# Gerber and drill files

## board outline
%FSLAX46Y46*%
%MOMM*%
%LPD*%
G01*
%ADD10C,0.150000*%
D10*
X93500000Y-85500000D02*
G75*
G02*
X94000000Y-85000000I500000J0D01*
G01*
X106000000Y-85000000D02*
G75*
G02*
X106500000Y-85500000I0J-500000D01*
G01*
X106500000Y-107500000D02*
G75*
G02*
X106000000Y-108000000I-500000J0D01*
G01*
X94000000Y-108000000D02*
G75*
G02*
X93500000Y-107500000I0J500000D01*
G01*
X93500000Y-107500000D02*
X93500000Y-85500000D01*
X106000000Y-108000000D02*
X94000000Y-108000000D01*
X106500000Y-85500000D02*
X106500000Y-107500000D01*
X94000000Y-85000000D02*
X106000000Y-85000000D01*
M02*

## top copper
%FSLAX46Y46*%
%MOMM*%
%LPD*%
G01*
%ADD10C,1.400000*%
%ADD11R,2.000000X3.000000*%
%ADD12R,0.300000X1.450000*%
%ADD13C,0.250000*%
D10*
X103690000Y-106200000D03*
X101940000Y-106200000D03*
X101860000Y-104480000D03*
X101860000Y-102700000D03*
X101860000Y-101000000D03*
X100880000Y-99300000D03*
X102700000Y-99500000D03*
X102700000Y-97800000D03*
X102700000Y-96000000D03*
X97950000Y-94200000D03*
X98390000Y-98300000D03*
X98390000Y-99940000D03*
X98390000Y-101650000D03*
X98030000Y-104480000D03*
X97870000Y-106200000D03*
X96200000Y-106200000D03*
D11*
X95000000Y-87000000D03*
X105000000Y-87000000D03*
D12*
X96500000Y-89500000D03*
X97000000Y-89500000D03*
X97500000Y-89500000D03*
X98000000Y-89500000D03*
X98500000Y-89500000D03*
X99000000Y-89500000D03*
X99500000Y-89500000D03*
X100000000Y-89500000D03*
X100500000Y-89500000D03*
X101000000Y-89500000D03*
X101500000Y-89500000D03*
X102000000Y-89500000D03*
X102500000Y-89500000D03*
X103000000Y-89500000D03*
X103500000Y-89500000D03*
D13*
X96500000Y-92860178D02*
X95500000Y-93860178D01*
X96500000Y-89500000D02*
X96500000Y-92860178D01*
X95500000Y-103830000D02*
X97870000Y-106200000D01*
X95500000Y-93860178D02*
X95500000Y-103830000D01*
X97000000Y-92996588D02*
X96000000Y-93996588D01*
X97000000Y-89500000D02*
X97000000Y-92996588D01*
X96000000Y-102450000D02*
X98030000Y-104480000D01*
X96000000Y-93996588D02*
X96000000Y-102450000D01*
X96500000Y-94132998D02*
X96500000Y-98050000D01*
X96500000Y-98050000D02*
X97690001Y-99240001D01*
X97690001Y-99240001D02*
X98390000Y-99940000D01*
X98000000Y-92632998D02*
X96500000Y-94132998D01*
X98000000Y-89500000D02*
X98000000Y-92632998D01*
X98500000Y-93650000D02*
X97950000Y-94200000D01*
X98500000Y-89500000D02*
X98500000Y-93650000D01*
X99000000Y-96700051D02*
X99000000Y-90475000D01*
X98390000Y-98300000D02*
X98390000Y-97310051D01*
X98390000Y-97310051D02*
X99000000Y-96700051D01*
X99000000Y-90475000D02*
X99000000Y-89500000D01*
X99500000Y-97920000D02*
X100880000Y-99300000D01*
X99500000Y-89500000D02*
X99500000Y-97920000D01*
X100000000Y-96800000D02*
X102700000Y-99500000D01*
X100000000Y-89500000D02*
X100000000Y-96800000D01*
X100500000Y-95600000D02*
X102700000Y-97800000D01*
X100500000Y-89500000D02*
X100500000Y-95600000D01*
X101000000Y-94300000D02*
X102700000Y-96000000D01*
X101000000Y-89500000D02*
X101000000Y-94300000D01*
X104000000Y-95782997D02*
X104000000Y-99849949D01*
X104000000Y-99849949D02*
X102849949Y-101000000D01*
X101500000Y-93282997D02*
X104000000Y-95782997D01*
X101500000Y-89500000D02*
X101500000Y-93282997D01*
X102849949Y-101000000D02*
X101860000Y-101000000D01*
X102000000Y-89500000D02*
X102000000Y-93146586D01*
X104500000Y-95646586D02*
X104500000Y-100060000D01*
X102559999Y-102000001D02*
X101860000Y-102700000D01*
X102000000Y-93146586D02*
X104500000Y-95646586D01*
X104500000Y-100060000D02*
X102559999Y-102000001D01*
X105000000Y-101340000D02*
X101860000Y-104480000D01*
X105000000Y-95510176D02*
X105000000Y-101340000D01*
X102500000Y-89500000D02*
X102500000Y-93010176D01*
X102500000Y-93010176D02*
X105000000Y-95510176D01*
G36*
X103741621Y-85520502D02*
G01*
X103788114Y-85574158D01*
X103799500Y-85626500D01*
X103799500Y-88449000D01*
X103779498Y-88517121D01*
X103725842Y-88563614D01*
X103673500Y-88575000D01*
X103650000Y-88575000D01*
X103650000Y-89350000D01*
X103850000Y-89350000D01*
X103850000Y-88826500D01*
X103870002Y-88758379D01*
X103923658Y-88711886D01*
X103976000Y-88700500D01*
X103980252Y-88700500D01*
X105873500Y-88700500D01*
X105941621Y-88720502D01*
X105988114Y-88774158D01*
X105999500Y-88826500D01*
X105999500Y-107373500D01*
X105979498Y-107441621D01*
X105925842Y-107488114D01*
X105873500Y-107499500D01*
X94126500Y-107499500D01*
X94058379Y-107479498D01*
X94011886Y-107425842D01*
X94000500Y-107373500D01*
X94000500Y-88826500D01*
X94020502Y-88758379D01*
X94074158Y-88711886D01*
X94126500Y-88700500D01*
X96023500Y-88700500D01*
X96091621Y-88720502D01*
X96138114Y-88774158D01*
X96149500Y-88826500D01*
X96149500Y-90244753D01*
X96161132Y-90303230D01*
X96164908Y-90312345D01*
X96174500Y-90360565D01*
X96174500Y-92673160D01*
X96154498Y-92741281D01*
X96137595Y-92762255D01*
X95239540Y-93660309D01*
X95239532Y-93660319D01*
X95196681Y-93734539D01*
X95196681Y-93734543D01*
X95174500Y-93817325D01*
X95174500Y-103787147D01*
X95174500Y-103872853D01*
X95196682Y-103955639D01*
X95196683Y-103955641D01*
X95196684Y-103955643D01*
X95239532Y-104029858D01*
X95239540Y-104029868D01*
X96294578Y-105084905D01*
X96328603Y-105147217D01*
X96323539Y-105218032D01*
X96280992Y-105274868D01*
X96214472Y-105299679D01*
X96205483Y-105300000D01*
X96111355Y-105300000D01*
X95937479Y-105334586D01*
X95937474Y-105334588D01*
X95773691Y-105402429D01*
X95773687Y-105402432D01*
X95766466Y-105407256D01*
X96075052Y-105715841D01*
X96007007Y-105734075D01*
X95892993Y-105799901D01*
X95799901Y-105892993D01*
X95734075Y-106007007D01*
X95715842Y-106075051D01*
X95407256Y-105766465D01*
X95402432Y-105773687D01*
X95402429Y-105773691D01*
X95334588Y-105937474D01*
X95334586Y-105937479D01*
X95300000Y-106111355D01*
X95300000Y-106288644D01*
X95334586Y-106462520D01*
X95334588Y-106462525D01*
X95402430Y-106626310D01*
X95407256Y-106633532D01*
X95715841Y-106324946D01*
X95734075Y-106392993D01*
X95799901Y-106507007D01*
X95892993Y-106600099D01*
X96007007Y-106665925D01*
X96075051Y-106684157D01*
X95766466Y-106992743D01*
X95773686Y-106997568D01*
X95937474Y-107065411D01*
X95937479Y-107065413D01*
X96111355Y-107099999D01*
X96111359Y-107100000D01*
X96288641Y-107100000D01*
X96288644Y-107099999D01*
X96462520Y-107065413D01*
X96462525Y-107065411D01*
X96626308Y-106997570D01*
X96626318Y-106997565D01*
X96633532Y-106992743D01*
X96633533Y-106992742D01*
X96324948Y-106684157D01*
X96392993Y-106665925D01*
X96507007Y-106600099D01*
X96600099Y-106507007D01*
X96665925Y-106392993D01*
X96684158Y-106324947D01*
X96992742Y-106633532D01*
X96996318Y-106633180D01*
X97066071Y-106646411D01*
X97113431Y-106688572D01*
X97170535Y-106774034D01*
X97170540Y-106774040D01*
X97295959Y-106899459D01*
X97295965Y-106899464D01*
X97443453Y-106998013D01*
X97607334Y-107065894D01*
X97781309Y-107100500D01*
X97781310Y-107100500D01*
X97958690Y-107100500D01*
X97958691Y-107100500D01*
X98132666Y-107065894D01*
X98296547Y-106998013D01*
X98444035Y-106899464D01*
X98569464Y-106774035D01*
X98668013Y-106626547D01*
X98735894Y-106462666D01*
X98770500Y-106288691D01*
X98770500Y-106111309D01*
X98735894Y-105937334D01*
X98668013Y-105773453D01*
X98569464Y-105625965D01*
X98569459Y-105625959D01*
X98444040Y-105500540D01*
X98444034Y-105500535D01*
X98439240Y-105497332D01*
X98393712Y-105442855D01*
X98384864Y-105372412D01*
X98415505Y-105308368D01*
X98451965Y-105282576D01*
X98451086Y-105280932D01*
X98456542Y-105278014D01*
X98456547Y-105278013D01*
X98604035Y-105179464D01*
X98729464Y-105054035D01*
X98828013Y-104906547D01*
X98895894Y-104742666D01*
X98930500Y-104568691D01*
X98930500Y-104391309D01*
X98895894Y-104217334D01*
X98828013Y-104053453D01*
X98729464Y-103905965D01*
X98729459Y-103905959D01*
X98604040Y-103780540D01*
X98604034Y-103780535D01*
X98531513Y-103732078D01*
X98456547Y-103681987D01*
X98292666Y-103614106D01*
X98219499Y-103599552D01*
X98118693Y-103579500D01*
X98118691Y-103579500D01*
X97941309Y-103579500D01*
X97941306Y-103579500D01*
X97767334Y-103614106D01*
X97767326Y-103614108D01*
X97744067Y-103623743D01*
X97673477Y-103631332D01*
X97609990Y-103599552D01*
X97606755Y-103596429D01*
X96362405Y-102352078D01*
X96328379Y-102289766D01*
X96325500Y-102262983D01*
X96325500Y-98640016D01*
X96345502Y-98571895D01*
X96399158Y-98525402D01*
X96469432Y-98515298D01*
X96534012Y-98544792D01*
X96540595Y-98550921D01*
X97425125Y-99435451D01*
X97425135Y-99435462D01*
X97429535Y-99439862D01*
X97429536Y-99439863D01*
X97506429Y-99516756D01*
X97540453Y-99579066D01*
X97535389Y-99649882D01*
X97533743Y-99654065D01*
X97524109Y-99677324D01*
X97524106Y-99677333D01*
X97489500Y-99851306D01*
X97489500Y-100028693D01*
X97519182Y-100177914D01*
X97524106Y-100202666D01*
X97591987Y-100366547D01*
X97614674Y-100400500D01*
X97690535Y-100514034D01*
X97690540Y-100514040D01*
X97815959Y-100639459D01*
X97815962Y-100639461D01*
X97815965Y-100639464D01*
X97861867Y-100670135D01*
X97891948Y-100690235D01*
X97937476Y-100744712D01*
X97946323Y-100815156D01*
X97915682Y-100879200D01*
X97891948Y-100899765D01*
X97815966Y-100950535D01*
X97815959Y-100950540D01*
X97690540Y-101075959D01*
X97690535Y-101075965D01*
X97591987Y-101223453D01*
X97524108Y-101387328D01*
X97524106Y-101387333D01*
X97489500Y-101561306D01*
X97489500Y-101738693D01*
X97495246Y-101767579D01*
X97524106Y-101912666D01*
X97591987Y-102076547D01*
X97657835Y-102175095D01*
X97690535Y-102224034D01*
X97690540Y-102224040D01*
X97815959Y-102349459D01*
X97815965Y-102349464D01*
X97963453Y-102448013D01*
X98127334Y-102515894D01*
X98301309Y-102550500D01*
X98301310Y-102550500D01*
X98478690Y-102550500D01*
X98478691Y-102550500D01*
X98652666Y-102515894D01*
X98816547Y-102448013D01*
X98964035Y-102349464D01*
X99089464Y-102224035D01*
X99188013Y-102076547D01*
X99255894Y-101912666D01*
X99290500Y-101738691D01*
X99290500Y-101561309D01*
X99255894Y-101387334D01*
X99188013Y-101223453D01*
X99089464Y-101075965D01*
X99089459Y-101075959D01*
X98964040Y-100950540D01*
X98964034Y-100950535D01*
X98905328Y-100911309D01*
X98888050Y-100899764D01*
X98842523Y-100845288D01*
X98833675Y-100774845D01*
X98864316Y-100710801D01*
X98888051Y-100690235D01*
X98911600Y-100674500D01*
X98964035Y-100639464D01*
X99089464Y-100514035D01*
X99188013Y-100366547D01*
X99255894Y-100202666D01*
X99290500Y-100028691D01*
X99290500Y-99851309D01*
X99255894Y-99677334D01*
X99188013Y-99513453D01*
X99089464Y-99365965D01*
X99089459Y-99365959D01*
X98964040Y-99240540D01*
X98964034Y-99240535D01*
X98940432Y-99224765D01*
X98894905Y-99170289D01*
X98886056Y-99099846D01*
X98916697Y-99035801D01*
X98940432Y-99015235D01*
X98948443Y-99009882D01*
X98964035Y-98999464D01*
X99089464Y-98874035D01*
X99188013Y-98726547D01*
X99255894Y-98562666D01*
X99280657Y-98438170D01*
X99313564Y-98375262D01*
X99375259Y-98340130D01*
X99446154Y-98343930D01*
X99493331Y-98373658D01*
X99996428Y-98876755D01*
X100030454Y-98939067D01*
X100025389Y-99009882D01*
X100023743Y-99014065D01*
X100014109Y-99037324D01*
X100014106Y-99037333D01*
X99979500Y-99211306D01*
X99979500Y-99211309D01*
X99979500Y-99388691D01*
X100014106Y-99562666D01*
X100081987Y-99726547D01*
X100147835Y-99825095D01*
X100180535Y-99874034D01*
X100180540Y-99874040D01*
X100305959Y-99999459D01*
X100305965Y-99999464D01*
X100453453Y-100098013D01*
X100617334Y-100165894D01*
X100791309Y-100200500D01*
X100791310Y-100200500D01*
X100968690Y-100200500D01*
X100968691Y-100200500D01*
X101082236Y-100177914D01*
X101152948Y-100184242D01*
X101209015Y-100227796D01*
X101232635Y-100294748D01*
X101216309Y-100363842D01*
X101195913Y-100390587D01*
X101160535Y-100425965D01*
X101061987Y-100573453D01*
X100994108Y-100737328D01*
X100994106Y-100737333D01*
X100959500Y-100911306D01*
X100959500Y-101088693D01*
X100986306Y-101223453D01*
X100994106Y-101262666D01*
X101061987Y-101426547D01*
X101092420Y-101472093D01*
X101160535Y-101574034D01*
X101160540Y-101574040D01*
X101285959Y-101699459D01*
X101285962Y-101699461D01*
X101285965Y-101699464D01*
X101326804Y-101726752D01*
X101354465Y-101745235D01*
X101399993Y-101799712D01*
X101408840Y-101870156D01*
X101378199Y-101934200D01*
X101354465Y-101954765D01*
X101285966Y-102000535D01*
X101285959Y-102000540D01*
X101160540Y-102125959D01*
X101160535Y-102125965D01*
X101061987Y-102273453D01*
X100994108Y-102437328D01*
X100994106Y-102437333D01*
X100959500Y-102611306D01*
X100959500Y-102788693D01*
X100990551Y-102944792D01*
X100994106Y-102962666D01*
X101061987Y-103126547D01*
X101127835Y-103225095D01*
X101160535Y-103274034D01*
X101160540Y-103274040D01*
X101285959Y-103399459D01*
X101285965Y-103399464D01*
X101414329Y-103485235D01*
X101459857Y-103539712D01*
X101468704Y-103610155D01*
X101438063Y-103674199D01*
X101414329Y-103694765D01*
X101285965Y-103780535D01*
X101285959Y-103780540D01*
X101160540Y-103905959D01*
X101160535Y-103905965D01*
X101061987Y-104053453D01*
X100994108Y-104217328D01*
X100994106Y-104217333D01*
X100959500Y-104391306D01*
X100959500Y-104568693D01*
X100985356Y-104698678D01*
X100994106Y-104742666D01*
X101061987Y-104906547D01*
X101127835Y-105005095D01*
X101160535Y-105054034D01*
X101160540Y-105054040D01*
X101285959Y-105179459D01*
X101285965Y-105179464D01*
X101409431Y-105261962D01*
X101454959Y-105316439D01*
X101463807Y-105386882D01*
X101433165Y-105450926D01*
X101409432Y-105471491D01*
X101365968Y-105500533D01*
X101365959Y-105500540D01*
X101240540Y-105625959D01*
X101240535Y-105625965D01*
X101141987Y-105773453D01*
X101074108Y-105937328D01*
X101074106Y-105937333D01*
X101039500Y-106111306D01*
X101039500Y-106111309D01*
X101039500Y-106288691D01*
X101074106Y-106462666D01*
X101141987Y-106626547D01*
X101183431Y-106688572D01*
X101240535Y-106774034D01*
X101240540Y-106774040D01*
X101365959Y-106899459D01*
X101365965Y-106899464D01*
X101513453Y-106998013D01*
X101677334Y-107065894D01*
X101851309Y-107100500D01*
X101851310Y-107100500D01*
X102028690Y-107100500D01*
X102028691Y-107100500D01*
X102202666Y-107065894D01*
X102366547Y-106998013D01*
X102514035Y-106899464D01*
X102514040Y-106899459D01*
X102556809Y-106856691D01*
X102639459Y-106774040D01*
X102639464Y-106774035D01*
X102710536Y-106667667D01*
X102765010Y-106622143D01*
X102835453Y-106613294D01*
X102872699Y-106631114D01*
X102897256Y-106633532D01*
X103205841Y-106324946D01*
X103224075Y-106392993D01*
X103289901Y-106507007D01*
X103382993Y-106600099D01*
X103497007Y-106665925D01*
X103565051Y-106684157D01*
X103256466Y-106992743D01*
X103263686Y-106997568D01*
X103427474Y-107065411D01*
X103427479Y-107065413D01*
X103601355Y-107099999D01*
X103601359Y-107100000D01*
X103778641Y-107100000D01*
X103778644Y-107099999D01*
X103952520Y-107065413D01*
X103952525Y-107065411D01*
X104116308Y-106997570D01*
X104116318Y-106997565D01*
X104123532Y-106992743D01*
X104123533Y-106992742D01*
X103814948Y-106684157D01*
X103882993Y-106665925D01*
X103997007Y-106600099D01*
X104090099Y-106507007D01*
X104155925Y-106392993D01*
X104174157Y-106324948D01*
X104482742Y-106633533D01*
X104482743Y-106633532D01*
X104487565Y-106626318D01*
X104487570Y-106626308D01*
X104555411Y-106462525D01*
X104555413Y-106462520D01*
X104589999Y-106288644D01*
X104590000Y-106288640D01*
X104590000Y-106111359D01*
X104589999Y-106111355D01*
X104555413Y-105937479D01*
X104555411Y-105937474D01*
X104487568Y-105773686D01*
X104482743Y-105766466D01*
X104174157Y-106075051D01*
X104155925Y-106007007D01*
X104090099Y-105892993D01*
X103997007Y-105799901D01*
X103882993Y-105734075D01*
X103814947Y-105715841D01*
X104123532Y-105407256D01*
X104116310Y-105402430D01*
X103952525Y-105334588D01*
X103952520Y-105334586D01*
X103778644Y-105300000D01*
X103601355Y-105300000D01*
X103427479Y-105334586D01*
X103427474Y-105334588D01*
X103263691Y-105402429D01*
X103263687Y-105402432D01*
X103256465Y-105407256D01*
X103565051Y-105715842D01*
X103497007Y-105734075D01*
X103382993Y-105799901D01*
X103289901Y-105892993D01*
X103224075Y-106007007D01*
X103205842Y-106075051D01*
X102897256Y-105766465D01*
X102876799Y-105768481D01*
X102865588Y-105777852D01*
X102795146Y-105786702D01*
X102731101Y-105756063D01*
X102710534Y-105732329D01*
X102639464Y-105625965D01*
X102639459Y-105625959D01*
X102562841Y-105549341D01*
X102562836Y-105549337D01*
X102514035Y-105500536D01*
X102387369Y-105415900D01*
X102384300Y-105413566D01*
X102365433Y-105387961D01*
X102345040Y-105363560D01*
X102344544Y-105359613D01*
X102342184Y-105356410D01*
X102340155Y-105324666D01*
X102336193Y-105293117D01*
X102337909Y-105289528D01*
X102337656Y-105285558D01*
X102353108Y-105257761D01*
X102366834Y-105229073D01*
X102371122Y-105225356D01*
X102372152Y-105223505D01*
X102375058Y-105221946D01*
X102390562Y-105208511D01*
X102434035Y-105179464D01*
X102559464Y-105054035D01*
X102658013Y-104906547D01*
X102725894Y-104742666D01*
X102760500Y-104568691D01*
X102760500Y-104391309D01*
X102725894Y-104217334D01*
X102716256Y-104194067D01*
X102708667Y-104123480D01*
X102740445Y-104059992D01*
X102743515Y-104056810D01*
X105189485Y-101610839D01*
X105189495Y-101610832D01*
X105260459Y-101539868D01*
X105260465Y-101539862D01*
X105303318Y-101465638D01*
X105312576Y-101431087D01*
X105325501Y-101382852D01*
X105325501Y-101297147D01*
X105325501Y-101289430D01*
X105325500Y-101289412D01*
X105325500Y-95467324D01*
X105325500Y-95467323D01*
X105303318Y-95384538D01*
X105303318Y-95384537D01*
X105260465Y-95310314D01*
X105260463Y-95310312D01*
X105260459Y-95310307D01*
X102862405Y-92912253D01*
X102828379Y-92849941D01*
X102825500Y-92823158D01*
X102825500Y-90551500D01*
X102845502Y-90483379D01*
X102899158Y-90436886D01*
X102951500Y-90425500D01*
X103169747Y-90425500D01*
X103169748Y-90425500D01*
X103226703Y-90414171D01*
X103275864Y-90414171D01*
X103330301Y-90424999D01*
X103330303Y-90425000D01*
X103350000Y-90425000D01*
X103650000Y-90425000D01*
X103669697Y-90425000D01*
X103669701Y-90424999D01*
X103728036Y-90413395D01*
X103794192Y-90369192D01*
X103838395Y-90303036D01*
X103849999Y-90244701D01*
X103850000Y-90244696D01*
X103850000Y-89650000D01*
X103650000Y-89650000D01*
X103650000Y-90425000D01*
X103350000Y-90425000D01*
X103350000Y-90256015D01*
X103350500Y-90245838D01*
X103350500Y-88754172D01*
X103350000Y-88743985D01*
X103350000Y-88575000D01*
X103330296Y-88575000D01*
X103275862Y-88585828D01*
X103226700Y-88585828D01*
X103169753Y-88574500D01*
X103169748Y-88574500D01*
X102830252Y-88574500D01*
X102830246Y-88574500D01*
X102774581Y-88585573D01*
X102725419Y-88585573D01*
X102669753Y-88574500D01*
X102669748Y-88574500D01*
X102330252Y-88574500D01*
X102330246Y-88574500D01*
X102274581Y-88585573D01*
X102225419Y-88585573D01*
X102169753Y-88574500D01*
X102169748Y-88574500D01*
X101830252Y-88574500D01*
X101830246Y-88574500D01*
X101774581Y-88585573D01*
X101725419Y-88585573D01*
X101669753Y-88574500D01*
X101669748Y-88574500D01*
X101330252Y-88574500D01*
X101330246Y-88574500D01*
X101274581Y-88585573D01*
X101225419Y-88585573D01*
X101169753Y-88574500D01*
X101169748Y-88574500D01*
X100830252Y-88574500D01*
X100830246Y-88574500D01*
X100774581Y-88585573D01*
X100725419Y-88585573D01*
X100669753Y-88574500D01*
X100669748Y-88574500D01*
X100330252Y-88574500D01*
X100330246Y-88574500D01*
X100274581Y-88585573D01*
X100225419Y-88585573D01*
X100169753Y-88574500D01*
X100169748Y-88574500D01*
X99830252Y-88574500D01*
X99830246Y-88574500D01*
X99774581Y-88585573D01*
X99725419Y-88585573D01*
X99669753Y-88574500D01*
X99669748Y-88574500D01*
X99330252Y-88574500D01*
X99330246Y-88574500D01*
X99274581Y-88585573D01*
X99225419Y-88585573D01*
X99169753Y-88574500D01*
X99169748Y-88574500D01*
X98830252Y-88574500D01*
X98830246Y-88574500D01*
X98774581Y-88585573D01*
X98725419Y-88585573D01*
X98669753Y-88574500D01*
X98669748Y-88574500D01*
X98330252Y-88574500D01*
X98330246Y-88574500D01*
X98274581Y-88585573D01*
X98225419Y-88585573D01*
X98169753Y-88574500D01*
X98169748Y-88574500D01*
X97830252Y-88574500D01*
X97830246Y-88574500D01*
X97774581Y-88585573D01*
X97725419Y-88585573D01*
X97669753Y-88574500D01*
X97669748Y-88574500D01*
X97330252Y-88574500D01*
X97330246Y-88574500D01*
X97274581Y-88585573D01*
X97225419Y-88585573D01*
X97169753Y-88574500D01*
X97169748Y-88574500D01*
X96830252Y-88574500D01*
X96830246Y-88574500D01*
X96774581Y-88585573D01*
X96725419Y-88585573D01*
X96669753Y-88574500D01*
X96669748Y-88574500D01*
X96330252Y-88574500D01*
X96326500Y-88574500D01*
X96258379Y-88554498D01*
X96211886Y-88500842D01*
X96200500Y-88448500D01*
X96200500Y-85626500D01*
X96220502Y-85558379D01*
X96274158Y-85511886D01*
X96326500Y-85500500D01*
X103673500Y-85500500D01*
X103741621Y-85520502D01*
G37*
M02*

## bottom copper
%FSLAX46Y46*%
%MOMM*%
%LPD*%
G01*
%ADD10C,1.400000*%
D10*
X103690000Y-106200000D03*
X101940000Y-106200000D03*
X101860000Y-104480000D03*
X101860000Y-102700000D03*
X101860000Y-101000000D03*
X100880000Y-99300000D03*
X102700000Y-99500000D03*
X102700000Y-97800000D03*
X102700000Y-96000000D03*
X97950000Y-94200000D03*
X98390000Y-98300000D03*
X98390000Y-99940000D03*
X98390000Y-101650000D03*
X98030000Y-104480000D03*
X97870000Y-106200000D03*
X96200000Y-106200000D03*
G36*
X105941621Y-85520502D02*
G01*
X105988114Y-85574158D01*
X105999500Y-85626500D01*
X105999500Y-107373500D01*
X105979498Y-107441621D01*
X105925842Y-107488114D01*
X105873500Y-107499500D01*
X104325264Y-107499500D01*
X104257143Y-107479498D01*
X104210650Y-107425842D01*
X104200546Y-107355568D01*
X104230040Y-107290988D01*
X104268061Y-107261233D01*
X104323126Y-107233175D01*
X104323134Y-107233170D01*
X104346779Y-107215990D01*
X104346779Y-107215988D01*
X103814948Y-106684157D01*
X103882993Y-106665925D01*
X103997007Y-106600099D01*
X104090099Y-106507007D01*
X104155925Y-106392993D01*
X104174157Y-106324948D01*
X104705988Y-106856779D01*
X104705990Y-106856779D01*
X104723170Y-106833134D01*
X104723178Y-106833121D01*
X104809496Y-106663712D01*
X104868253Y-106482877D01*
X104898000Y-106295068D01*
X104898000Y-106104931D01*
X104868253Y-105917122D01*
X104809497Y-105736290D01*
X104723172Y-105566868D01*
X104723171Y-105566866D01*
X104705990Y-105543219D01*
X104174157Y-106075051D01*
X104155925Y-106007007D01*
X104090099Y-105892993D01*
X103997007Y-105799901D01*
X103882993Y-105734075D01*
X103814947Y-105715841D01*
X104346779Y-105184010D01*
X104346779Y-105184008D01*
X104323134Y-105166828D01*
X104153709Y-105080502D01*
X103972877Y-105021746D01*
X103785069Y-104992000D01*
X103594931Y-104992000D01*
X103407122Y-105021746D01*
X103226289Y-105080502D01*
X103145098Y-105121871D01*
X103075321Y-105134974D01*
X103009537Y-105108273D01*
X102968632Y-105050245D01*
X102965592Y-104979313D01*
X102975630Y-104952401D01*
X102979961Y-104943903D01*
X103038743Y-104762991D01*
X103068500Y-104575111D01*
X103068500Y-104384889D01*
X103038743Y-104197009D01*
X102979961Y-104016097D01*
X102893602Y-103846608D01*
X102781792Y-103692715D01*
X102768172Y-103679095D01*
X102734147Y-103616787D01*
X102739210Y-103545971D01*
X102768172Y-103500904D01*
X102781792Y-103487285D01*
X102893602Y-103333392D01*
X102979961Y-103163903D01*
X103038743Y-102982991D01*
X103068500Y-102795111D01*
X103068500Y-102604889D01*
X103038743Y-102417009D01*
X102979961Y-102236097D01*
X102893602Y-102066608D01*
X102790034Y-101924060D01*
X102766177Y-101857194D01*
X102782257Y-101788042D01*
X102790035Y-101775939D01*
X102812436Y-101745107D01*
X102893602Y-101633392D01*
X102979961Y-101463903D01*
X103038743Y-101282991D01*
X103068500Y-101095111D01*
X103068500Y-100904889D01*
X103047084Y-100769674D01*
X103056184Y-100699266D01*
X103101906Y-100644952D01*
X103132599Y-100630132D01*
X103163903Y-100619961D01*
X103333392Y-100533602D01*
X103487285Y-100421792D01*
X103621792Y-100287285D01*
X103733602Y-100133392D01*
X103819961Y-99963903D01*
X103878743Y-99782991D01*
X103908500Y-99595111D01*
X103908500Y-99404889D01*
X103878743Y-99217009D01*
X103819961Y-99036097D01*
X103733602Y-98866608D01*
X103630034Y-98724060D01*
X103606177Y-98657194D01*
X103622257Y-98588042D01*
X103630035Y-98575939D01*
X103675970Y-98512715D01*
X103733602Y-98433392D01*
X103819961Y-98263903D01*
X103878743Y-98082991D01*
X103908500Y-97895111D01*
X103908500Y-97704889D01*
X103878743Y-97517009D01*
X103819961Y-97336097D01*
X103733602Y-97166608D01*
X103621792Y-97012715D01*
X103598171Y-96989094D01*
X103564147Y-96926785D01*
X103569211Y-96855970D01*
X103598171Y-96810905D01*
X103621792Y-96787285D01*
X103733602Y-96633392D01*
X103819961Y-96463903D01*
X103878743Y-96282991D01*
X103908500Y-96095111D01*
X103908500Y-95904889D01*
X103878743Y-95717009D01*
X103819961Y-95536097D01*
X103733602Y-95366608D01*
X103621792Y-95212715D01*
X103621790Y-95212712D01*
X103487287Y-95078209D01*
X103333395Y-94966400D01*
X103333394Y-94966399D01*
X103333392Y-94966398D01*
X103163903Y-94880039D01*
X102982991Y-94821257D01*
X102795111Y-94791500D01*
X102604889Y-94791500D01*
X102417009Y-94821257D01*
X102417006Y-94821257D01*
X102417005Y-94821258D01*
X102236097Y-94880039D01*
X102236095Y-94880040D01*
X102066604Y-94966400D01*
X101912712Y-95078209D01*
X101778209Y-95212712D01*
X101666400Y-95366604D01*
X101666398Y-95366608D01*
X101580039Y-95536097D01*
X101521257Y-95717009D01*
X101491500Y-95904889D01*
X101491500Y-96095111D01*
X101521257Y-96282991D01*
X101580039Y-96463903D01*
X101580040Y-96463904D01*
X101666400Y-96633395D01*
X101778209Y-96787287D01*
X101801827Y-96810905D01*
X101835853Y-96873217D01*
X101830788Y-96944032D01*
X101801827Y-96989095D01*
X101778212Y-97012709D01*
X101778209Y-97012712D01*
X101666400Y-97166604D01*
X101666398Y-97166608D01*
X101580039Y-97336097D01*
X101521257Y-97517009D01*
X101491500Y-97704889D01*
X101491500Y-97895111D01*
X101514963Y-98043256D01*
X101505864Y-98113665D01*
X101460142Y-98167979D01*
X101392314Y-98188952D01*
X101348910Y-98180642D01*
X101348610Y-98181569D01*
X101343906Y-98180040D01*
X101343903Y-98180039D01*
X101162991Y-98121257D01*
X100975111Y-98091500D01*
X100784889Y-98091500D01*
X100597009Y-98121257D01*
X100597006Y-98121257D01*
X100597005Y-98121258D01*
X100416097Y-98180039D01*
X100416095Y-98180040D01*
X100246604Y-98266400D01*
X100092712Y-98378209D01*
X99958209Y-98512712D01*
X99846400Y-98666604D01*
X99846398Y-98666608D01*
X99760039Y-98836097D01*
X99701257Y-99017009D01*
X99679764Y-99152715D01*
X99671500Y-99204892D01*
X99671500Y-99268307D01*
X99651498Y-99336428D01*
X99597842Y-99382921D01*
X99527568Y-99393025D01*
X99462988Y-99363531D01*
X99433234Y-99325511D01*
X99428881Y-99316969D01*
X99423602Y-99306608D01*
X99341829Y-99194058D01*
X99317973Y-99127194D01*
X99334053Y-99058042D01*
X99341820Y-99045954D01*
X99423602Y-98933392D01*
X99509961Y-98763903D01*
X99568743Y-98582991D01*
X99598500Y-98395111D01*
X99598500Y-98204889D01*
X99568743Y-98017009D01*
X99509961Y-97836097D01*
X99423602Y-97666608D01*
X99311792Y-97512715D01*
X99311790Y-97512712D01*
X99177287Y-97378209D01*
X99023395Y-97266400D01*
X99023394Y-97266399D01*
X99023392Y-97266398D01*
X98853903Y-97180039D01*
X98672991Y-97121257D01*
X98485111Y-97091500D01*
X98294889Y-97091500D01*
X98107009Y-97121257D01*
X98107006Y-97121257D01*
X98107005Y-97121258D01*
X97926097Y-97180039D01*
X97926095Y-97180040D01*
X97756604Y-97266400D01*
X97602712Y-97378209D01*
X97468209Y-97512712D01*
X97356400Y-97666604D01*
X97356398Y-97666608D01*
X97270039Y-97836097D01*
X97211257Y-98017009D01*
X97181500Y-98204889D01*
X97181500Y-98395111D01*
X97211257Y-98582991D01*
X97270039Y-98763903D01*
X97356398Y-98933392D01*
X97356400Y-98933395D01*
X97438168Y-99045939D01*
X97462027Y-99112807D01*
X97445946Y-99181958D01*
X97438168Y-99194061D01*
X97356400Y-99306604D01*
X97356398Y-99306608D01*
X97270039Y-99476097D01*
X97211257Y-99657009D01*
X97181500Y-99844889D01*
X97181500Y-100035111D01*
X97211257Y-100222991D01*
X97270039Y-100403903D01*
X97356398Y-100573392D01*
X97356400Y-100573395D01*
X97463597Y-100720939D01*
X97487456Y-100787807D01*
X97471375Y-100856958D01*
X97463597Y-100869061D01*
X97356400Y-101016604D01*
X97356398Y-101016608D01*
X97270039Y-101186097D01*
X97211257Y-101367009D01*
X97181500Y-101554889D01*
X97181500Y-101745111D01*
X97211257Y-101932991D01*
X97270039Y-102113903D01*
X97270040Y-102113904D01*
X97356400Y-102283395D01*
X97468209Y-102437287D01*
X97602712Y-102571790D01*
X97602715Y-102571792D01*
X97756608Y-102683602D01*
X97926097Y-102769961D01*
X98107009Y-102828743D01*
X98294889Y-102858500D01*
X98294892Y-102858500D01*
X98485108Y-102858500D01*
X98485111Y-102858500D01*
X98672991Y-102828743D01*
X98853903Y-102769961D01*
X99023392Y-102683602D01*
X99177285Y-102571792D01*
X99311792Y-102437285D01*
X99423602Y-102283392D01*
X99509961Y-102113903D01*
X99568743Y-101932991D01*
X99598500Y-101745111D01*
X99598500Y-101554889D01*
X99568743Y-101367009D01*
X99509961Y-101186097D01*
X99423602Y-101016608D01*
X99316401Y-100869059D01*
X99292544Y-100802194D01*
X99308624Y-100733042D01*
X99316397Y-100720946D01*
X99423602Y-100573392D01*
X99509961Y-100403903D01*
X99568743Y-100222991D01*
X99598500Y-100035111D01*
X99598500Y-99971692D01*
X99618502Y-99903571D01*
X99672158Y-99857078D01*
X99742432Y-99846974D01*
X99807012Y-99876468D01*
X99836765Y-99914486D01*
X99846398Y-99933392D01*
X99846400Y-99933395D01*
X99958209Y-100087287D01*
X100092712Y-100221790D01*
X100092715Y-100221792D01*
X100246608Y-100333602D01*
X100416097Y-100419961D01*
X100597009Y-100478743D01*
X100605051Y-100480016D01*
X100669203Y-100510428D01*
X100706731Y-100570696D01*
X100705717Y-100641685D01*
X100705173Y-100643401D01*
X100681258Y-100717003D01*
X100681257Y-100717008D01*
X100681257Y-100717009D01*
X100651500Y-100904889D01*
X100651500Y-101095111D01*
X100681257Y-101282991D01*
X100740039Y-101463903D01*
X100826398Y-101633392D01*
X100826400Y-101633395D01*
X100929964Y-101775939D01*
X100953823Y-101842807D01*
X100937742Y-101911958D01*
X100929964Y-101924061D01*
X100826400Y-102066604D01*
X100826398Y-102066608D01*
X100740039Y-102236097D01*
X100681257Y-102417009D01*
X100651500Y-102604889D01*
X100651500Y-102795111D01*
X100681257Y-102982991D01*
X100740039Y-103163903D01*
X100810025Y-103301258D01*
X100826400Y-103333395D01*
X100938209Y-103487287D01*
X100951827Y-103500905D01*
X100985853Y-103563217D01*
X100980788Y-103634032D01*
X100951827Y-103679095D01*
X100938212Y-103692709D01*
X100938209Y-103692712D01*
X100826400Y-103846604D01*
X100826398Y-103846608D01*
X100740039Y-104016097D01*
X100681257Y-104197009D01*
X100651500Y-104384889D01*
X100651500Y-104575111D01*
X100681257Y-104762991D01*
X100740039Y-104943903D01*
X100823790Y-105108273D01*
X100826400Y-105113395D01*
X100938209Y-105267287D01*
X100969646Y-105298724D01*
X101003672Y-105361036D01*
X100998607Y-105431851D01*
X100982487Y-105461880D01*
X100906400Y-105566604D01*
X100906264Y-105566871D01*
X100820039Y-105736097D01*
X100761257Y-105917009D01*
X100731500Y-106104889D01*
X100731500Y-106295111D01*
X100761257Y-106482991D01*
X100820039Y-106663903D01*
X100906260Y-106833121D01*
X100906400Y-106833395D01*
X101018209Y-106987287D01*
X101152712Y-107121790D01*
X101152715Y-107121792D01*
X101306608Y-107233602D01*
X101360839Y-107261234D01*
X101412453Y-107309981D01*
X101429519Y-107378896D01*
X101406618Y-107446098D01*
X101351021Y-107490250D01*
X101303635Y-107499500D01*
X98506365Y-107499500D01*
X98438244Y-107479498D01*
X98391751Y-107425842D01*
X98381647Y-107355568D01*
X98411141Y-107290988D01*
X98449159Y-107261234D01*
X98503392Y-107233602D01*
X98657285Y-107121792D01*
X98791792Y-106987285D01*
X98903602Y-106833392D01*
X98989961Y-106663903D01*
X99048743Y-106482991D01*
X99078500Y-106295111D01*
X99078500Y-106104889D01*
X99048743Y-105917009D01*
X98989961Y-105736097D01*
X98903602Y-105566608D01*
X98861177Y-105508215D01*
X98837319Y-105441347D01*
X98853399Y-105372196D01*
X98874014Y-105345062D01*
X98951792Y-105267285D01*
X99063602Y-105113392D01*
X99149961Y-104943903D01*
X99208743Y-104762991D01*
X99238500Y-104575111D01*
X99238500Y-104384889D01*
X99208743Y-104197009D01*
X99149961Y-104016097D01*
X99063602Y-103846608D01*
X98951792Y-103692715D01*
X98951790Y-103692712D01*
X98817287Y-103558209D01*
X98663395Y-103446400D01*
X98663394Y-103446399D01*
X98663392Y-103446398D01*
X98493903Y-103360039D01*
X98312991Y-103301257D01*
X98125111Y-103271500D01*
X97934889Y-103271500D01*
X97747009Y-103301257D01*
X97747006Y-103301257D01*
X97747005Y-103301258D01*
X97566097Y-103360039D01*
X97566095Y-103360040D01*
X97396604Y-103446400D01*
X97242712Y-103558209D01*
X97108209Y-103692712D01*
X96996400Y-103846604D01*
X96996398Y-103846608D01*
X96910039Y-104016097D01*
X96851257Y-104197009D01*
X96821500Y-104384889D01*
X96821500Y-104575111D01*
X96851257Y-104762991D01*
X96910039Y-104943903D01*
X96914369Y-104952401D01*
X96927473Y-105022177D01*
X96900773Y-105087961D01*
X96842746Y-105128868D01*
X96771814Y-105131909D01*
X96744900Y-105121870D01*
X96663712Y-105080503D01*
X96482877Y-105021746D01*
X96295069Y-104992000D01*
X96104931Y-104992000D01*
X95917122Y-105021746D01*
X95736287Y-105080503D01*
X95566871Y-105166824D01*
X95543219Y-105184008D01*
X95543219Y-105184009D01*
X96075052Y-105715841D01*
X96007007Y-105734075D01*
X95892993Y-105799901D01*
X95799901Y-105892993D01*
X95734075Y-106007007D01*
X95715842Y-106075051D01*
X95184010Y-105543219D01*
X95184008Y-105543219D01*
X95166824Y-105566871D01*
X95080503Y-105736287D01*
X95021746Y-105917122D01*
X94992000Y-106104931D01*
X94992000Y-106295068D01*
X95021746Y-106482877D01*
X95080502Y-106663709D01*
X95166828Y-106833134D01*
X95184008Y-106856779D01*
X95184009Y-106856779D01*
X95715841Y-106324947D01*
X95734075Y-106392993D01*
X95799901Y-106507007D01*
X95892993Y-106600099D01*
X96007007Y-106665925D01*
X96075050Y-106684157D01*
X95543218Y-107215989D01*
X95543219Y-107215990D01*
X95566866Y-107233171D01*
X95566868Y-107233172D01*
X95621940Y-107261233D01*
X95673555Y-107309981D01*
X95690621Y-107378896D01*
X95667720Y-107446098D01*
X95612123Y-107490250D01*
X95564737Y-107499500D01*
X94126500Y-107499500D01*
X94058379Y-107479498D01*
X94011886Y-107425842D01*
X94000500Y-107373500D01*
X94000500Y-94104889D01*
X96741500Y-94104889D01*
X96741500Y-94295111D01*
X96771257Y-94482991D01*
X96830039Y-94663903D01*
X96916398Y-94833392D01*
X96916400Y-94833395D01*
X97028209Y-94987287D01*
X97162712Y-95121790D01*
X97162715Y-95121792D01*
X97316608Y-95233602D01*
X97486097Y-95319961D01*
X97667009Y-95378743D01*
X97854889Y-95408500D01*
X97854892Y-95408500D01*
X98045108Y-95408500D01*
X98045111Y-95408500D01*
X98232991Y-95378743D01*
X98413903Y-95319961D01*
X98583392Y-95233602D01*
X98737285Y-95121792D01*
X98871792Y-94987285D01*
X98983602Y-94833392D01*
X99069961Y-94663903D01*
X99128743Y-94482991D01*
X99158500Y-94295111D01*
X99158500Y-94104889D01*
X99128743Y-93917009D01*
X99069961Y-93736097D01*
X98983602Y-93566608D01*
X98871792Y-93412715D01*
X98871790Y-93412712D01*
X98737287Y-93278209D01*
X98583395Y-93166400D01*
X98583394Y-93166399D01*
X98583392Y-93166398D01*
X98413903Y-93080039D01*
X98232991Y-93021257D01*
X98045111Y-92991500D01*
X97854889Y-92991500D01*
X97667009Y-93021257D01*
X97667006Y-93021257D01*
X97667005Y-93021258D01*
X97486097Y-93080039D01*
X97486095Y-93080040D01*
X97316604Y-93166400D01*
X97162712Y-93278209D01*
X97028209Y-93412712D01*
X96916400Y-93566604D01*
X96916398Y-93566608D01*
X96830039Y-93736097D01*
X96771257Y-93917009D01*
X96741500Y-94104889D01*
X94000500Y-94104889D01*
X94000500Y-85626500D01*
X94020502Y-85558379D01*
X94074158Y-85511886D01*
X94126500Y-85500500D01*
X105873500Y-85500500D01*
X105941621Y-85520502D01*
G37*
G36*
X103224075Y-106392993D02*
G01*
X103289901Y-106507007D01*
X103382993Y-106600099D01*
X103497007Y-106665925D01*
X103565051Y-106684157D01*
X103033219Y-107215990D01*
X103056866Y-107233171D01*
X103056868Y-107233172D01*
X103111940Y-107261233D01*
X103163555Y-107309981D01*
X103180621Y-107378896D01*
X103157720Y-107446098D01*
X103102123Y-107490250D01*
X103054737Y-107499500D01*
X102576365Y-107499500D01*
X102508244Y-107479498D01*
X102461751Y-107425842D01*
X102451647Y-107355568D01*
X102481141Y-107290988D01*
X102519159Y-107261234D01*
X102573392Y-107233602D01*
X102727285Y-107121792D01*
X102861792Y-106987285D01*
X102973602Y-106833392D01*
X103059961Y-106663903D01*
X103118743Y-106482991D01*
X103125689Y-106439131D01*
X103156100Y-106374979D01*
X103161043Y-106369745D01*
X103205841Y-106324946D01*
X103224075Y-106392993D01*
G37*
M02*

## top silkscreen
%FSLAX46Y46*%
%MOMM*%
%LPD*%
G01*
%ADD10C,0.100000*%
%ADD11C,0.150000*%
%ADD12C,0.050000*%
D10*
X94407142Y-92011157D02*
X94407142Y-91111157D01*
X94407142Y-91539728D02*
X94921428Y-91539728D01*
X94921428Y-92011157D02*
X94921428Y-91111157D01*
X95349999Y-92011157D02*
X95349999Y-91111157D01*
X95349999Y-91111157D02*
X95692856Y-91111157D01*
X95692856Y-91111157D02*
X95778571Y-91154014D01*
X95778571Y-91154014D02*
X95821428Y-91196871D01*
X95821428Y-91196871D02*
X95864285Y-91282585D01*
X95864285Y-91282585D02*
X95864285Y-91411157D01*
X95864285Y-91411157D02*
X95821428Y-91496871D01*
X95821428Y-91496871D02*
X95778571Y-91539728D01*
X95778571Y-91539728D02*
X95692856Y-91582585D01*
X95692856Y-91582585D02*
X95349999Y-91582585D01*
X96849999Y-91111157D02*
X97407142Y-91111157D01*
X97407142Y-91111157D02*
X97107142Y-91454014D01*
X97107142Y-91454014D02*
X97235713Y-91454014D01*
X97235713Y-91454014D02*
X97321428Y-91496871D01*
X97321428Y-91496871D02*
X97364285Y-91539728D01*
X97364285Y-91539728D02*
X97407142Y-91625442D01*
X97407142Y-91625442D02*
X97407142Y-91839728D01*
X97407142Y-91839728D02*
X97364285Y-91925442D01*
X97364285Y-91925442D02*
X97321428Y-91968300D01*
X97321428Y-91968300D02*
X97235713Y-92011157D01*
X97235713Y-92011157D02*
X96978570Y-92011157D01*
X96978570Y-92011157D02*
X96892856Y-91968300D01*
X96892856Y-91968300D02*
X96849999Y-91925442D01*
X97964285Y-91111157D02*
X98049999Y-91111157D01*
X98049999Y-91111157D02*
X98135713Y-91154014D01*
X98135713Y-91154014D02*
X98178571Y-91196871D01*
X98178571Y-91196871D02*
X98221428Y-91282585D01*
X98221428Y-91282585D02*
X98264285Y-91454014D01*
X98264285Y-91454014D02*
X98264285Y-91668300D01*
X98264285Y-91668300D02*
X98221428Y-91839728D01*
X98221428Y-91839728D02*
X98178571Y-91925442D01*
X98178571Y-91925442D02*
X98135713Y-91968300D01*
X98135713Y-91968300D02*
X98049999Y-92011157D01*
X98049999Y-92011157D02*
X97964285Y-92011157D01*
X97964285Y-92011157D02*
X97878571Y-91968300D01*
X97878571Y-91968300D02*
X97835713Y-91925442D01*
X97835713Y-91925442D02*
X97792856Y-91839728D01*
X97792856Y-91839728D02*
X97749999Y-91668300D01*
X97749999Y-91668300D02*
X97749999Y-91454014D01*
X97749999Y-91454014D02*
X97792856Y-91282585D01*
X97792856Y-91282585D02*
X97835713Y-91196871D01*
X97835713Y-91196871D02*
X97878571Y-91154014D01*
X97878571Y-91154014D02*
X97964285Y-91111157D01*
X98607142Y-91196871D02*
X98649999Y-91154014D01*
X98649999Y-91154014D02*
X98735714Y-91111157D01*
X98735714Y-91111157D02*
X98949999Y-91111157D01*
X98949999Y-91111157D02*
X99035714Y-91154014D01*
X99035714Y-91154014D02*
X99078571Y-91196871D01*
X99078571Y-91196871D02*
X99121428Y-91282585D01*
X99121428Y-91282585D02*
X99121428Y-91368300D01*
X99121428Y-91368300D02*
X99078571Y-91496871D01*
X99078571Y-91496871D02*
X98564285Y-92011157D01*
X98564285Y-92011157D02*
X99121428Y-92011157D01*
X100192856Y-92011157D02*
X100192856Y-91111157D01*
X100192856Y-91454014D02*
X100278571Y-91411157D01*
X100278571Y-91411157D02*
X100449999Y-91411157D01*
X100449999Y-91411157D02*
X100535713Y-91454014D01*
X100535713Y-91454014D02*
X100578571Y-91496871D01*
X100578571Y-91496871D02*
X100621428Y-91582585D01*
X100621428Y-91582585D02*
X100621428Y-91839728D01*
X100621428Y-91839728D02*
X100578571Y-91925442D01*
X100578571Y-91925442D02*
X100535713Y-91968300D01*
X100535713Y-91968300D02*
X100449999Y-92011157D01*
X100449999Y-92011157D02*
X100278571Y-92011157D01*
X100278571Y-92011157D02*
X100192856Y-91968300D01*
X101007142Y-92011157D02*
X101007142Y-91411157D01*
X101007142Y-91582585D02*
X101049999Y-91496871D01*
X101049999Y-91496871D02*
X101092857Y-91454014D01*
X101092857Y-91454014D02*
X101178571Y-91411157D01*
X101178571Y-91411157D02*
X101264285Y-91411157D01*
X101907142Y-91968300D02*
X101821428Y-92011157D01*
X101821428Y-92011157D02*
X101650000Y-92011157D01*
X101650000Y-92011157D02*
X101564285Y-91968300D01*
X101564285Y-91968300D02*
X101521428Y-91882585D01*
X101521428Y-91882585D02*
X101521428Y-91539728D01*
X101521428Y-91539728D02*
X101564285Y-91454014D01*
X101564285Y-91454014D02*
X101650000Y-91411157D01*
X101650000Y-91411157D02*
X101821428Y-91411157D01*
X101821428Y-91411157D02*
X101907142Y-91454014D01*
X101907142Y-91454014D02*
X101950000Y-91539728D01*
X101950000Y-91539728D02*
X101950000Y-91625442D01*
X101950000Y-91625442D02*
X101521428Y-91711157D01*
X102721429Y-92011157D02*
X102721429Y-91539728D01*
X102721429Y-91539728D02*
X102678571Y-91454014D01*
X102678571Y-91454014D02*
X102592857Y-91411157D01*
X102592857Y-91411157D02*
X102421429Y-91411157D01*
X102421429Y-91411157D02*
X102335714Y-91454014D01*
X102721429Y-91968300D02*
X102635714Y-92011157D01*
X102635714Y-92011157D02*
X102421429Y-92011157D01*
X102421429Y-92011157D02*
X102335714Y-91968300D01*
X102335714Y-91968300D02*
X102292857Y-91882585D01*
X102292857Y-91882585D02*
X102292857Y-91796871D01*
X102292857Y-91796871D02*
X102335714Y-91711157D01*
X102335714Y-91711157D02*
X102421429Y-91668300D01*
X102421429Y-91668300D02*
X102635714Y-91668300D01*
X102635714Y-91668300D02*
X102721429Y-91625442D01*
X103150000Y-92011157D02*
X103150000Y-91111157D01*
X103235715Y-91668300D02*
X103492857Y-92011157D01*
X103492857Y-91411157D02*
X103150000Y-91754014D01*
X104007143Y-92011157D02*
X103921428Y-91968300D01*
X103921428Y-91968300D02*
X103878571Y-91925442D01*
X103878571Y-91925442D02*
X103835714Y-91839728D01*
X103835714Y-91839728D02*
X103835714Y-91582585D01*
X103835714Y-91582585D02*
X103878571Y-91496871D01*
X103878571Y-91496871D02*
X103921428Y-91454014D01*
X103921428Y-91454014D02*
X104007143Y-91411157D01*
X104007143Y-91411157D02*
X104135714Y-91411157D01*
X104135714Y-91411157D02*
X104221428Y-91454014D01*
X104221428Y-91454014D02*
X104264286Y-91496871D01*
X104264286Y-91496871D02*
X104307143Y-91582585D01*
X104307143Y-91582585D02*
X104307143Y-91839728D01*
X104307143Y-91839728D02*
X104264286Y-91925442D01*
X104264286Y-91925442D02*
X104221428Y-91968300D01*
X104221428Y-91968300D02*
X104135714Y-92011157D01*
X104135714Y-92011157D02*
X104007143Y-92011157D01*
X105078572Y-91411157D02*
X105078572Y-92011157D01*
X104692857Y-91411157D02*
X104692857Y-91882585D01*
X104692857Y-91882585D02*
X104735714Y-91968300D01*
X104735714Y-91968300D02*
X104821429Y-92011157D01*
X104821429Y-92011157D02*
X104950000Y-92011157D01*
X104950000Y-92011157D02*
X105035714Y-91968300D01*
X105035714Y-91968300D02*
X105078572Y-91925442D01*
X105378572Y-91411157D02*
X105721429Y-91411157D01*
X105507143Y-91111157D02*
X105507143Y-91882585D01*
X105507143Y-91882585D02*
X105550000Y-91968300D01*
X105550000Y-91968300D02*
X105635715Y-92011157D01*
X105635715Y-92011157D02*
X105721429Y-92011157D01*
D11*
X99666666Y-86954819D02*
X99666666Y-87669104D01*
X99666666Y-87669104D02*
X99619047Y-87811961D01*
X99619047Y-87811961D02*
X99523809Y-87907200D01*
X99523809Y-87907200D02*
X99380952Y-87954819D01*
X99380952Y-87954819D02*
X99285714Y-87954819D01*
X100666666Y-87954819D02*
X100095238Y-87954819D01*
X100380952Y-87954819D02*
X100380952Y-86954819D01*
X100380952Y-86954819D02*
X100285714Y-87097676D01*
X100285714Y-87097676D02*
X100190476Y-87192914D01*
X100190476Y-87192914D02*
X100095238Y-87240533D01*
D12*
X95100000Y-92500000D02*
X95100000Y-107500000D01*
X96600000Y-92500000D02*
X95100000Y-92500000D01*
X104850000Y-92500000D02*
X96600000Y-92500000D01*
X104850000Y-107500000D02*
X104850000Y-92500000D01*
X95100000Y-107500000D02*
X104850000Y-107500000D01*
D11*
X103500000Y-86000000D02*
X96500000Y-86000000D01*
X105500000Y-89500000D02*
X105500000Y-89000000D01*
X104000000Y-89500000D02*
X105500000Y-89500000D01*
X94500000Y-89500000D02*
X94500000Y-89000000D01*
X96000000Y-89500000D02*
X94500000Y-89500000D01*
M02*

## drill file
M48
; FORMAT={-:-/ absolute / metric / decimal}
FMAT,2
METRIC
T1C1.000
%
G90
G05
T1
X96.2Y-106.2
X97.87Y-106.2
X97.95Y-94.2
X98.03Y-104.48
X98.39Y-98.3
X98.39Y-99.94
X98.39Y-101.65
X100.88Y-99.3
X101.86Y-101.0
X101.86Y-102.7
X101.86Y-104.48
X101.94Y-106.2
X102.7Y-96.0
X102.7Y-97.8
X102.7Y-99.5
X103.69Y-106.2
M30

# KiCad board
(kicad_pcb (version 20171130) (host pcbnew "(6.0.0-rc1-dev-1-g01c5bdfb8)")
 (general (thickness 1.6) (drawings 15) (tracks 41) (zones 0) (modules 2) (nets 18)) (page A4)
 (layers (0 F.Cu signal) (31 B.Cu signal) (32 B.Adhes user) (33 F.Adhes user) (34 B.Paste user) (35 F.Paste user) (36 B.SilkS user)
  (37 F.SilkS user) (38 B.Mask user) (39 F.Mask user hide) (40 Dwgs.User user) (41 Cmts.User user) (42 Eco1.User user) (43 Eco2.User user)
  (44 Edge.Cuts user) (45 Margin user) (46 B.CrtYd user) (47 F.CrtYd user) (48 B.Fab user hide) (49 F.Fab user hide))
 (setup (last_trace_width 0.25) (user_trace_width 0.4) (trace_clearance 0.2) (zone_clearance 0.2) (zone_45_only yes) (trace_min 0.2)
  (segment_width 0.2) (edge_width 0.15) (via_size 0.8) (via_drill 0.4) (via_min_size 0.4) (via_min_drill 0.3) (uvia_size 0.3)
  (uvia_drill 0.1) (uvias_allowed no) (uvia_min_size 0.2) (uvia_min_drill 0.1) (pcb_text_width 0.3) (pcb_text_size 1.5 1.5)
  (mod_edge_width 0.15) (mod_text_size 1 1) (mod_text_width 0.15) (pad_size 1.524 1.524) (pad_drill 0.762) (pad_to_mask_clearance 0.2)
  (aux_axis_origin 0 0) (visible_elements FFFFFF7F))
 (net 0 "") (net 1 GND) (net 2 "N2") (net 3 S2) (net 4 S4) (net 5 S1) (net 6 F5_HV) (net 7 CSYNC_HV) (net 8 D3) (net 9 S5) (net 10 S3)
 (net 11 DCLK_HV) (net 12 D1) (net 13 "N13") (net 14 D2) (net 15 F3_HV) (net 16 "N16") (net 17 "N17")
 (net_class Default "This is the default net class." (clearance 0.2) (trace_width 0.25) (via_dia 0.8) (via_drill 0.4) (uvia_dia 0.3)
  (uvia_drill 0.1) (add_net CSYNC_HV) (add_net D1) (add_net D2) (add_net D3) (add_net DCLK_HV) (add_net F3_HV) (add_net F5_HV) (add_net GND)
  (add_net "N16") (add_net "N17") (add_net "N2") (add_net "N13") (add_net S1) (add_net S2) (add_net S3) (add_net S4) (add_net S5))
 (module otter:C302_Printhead (layer F.Cu) (at 100.1 100)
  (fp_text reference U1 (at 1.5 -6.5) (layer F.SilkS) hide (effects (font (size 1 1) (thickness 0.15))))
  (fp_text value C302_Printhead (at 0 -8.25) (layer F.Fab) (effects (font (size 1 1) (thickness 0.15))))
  (fp_line (start -5 -7.5) (end -5 7.5) (layer F.SilkS) (width 0.05))
  (fp_line (start -3.5 -7.5) (end -5 -7.5) (layer F.SilkS) (width 0.05))
  (fp_line (start 4.75 -7.5) (end -3.5 -7.5) (layer F.SilkS) (width 0.05))
  (fp_line (start 4.75 7.5) (end 4.75 -7.5) (layer F.SilkS) (width 0.05))
  (fp_line (start -5 7.5) (end 4.75 7.5) (layer F.SilkS) (width 0.05))
  (pad GND thru_hole circle (at 3.59 6.2) (size 1.4 1.4) (drill 1) (layers *.Cu *.Mask) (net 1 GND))
  (pad ID thru_hole circle (at 1.84 6.2) (size 1.4 1.4) (drill 1) (layers *.Cu *.Mask) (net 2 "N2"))
  (pad S2 thru_hole circle (at 1.76 4.48) (size 1.4 1.4) (drill 1) (layers *.Cu *.Mask) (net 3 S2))
  (pad S4 thru_hole circle (at 1.76 2.7) (size 1.4 1.4) (drill 1) (layers *.Cu *.Mask) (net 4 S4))
  (pad S1 thru_hole circle (at 1.76 1) (size 1.4 1.4) (drill 1) (layers *.Cu *.Mask) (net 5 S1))
  (pad PWRB thru_hole circle (at 0.78 -0.7) (size 1.4 1.4) (drill 1) (layers *.Cu *.Mask) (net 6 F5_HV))
  (pad CSYNC thru_hole circle (at 2.6 -0.5) (size 1.4 1.4) (drill 1) (layers *.Cu *.Mask) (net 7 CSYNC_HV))
  (pad D3 thru_hole circle (at 2.6 -2.2) (size 1.4 1.4) (drill 1) (layers *.Cu *.Mask) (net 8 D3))
  (pad S5 thru_hole circle (at 2.6 -4) (size 1.4 1.4) (drill 1) (layers *.Cu *.Mask) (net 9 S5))
  (pad S3 thru_hole circle (at -2.15 -5.8) (size 1.4 1.4) (drill 1) (layers *.Cu *.Mask) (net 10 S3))
  (pad DCLK thru_hole circle (at -1.71 -1.7) (size 1.4 1.4) (drill 1) (layers *.Cu *.Mask) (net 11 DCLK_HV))
  (pad D1 thru_hole circle (at -1.71 -0.06) (size 1.4 1.4) (drill 1) (layers *.Cu *.Mask) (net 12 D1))
  (pad TS thru_hole circle (at -1.71 1.65) (size 1.4 1.4) (drill 1) (layers *.Cu *.Mask) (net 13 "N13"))
  (pad D2 thru_hole circle (at -2.07 4.48) (size 1.4 1.4) (drill 1) (layers *.Cu *.Mask) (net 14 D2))
  (pad PWRA thru_hole circle (at -2.23 6.2) (size 1.4 1.4) (drill 1) (layers *.Cu *.Mask) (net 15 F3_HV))
  (pad GND thru_hole circle (at -3.9 6.2) (size 1.4 1.4) (drill 1) (layers *.Cu *.Mask) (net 1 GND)))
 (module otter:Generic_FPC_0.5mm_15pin (layer F.Cu) (at 100 88 180)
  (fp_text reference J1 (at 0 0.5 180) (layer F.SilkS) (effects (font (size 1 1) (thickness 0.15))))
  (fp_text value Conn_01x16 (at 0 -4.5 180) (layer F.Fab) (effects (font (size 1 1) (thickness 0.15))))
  (fp_line (start -3.5 2) (end 3.5 2) (layer F.SilkS) (width 0.15))
  (fp_line (start -5.5 -1.5) (end -5.5 -1) (layer F.SilkS) (width 0.15))
  (fp_line (start -4 -1.5) (end -5.5 -1.5) (layer F.SilkS) (width 0.15))
  (fp_line (start 5.5 -1.5) (end 5.5 -1) (layer F.SilkS) (width 0.15))
  (fp_line (start 4 -1.5) (end 5.5 -1.5) (layer F.SilkS) (width 0.15))
  (pad MP smd rect (at 5 1 180) (size 2 3) (layers F.Cu F.Paste F.Mask))
  (pad MP smd rect (at -5 1 180) (size 2 3) (layers F.Cu F.Paste F.Mask))
  (pad 15 smd rect (at 3.5 -1.5 180) (size 0.3 1.45) (layers F.Cu F.Paste F.Mask) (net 15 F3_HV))
  (pad 14 smd rect (at 3 -1.5 180) (size 0.3 1.45) (layers F.Cu F.Paste F.Mask) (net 14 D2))
  (pad 13 smd rect (at 2.5 -1.5 180) (size 0.3 1.45) (layers F.Cu F.Paste F.Mask) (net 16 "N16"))
  (pad 12 smd rect (at 2 -1.5 180) (size 0.3 1.45) (layers F.Cu F.Paste F.Mask) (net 12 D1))
  (pad 11 smd rect (at 1.5 -1.5 180) (size 0.3 1.45) (layers F.Cu F.Paste F.Mask) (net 10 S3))
  (pad 10 smd rect (at 1 -1.5 180) (size 0.3 1.45) (layers F.Cu F.Paste F.Mask) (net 11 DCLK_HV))
  (pad 9 smd rect (at 0.5 -1.5 180) (size 0.3 1.45) (layers F.Cu F.Paste F.Mask) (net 6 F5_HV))
  (pad 8 smd rect (at 0 -1.5) (size 0.3 1.45) (layers F.Cu F.Paste F.Mask) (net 7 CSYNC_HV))
  (pad 7 smd rect (at -0.5 -1.5 180) (size 0.3 1.45) (layers F.Cu F.Paste F.Mask) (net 8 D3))
  (pad 6 smd rect (at -1 -1.5 180) (size 0.3 1.45) (layers F.Cu F.Paste F.Mask) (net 9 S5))
  (pad 5 smd rect (at -1.5 -1.5 180) (size 0.3 1.45) (layers F.Cu F.Paste F.Mask) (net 5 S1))
  (pad 4 smd rect (at -2 -1.5 180) (size 0.3 1.45) (layers F.Cu F.Paste F.Mask) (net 4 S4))
  (pad 3 smd rect (at -2.5 -1.5 180) (size 0.3 1.45) (layers F.Cu F.Paste F.Mask) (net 3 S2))
  (pad 2 smd rect (at -3 -1.5 180) (size 0.3 1.45) (layers F.Cu F.Paste F.Mask) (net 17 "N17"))
  (pad 1 smd rect (at -3.5 -1.5 180) (size 0.3 1.45) (layers F.Cu F.Paste F.Mask) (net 1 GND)))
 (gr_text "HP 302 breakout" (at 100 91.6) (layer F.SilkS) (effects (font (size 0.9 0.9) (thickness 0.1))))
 (gr_arc (start 94 85.5) (end 94 85) (angle -90) (layer Edge.Cuts) (width 0.15))
 (gr_arc (start 106 85.5) (end 106.5 85.5) (angle -90) (layer Edge.Cuts) (width 0.15))
 (gr_arc (start 106 107.5) (end 106 108) (angle -90) (layer Edge.Cuts) (width 0.15))
 (gr_arc (start 94 107.5) (end 93.5 107.5) (angle -90) (layer Edge.Cuts) (width 0.15))
 (gr_line (start 93.5 107.5) (end 93.5 85.5) (layer Edge.Cuts) (width 0.15))
 (gr_line (start 106 108) (end 94 108) (layer Edge.Cuts) (width 0.15))
 (gr_line (start 106.5 85.5) (end 106.5 107.5) (layer Edge.Cuts) (width 0.15))
 (gr_line (start 94 85) (end 106 85) (layer Edge.Cuts) (width 0.15))
 (segment (start 96.5 92.860178) (end 95.5 93.860178) (width 0.25) (layer F.Cu) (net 15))
 (segment (start 96.5 89.5) (end 96.5 92.860178) (width 0.25) (layer F.Cu) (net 15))
 (segment (start 95.5 103.83) (end 97.87 106.2) (width 0.25) (layer F.Cu) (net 15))
 (segment (start 95.5 93.860178) (end 95.5 103.83) (width 0.25) (layer F.Cu) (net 15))
 (segment (start 97 92.996588) (end 96 93.996588) (width 0.25) (layer F.Cu) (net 14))
 (segment (start 97 89.5) (end 97 92.996588) (width 0.25) (layer F.Cu) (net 14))
 (segment (start 96 102.45) (end 98.03 104.48) (width 0.25) (layer F.Cu) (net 14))
 (segment (start 96 93.996588) (end 96 102.45) (width 0.25) (layer F.Cu) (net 14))
 (segment (start 96.5 94.132998) (end 96.5 98.05) (width 0.25) (layer F.Cu) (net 12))
 (segment (start 96.5 98.05) (end 97.690001 99.240001) (width 0.25) (layer F.Cu) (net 12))
 (segment (start 97.690001 99.240001) (end 98.39 99.94) (width 0.25) (layer F.Cu) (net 12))
 (segment (start 98 92.632998) (end 96.5 94.132998) (width 0.25) (layer F.Cu) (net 12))
 (segment (start 98 89.5) (end 98 92.632998) (width 0.25) (layer F.Cu) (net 12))
 (segment (start 98.5 93.65) (end 97.95 94.2) (width 0.25) (layer F.Cu) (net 10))
 (segment (start 98.5 89.5) (end 98.5 93.65) (width 0.25) (layer F.Cu) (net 10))
 (segment (start 99 96.700051) (end 99 90.475) (width 0.25) (layer F.Cu) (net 11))
 (segment (start 98.39 98.3) (end 98.39 97.310051) (width 0.25) (layer F.Cu) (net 11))
 (segment (start 98.39 97.310051) (end 99 96.700051) (width 0.25) (layer F.Cu) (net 11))
 (segment (start 99 90.475) (end 99 89.5) (width 0.25) (layer F.Cu) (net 11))
 (segment (start 99.5 97.92) (end 100.88 99.3) (width 0.25) (layer F.Cu) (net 6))
 (segment (start 99.5 89.5) (end 99.5 97.92) (width 0.25) (layer F.Cu) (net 6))
 (segment (start 100 96.8) (end 102.7 99.5) (width 0.25) (layer F.Cu) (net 7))
 (segment (start 100 89.5) (end 100 96.8) (width 0.25) (layer F.Cu) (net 7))
 (segment (start 100.5 95.6) (end 102.7 97.8) (width 0.25) (layer F.Cu) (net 8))
 (segment (start 100.5 89.5) (end 100.5 95.6) (width 0.25) (layer F.Cu) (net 8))
 (segment (start 101 94.3) (end 102.7 96) (width 0.25) (layer F.Cu) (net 9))
 (segment (start 101 89.5) (end 101 94.3) (width 0.25) (layer F.Cu) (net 9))
 (segment (start 104 95.782997) (end 104 99.849949) (width 0.25) (layer F.Cu) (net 5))
 (segment (start 104 99.849949) (end 102.849949 101) (width 0.25) (layer F.Cu) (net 5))
 (segment (start 101.5 93.282997) (end 104 95.782997) (width 0.25) (layer F.Cu) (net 5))
 (segment (start 101.5 89.5) (end 101.5 93.282997) (width 0.25) (layer F.Cu) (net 5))
 (segment (start 102.849949 101) (end 101.86 101) (width 0.25) (layer F.Cu) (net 5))
 (segment (start 102 89.5) (end 102 93.146586) (width 0.25) (layer F.Cu) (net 4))
 (segment (start 104.5 95.646586) (end 104.5 100.06) (width 0.25) (layer F.Cu) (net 4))
 (segment (start 102.559999 102.000001) (end 101.86 102.7) (width 0.25) (layer F.Cu) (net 4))
 (segment (start 102 93.146586) (end 104.5 95.646586) (width 0.25) (layer F.Cu) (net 4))
 (segment (start 104.5 100.06) (end 102.559999 102.000001) (width 0.25) (layer F.Cu) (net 4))
 (segment (start 105 101.34) (end 101.86 104.48) (width 0.25) (layer F.Cu) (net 3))
 (segment (start 105 95.510176) (end 105 101.34) (width 0.25) (layer F.Cu) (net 3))
 (segment (start 102.5 89.5) (end 102.5 93.010176) (width 0.25) (layer F.Cu) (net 3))
 (segment (start 102.5 93.010176) (end 105 95.510176) (width 0.25) (layer F.Cu) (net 3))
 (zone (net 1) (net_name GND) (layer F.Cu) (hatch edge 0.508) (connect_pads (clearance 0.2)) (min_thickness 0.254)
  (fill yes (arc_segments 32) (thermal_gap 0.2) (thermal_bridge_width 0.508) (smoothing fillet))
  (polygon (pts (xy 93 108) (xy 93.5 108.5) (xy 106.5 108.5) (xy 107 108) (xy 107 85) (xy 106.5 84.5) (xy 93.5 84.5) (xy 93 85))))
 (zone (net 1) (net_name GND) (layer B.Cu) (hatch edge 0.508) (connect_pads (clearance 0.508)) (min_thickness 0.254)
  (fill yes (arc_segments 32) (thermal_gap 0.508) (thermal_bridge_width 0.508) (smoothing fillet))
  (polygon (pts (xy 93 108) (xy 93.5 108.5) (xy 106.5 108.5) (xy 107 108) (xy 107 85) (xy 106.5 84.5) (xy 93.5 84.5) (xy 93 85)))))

